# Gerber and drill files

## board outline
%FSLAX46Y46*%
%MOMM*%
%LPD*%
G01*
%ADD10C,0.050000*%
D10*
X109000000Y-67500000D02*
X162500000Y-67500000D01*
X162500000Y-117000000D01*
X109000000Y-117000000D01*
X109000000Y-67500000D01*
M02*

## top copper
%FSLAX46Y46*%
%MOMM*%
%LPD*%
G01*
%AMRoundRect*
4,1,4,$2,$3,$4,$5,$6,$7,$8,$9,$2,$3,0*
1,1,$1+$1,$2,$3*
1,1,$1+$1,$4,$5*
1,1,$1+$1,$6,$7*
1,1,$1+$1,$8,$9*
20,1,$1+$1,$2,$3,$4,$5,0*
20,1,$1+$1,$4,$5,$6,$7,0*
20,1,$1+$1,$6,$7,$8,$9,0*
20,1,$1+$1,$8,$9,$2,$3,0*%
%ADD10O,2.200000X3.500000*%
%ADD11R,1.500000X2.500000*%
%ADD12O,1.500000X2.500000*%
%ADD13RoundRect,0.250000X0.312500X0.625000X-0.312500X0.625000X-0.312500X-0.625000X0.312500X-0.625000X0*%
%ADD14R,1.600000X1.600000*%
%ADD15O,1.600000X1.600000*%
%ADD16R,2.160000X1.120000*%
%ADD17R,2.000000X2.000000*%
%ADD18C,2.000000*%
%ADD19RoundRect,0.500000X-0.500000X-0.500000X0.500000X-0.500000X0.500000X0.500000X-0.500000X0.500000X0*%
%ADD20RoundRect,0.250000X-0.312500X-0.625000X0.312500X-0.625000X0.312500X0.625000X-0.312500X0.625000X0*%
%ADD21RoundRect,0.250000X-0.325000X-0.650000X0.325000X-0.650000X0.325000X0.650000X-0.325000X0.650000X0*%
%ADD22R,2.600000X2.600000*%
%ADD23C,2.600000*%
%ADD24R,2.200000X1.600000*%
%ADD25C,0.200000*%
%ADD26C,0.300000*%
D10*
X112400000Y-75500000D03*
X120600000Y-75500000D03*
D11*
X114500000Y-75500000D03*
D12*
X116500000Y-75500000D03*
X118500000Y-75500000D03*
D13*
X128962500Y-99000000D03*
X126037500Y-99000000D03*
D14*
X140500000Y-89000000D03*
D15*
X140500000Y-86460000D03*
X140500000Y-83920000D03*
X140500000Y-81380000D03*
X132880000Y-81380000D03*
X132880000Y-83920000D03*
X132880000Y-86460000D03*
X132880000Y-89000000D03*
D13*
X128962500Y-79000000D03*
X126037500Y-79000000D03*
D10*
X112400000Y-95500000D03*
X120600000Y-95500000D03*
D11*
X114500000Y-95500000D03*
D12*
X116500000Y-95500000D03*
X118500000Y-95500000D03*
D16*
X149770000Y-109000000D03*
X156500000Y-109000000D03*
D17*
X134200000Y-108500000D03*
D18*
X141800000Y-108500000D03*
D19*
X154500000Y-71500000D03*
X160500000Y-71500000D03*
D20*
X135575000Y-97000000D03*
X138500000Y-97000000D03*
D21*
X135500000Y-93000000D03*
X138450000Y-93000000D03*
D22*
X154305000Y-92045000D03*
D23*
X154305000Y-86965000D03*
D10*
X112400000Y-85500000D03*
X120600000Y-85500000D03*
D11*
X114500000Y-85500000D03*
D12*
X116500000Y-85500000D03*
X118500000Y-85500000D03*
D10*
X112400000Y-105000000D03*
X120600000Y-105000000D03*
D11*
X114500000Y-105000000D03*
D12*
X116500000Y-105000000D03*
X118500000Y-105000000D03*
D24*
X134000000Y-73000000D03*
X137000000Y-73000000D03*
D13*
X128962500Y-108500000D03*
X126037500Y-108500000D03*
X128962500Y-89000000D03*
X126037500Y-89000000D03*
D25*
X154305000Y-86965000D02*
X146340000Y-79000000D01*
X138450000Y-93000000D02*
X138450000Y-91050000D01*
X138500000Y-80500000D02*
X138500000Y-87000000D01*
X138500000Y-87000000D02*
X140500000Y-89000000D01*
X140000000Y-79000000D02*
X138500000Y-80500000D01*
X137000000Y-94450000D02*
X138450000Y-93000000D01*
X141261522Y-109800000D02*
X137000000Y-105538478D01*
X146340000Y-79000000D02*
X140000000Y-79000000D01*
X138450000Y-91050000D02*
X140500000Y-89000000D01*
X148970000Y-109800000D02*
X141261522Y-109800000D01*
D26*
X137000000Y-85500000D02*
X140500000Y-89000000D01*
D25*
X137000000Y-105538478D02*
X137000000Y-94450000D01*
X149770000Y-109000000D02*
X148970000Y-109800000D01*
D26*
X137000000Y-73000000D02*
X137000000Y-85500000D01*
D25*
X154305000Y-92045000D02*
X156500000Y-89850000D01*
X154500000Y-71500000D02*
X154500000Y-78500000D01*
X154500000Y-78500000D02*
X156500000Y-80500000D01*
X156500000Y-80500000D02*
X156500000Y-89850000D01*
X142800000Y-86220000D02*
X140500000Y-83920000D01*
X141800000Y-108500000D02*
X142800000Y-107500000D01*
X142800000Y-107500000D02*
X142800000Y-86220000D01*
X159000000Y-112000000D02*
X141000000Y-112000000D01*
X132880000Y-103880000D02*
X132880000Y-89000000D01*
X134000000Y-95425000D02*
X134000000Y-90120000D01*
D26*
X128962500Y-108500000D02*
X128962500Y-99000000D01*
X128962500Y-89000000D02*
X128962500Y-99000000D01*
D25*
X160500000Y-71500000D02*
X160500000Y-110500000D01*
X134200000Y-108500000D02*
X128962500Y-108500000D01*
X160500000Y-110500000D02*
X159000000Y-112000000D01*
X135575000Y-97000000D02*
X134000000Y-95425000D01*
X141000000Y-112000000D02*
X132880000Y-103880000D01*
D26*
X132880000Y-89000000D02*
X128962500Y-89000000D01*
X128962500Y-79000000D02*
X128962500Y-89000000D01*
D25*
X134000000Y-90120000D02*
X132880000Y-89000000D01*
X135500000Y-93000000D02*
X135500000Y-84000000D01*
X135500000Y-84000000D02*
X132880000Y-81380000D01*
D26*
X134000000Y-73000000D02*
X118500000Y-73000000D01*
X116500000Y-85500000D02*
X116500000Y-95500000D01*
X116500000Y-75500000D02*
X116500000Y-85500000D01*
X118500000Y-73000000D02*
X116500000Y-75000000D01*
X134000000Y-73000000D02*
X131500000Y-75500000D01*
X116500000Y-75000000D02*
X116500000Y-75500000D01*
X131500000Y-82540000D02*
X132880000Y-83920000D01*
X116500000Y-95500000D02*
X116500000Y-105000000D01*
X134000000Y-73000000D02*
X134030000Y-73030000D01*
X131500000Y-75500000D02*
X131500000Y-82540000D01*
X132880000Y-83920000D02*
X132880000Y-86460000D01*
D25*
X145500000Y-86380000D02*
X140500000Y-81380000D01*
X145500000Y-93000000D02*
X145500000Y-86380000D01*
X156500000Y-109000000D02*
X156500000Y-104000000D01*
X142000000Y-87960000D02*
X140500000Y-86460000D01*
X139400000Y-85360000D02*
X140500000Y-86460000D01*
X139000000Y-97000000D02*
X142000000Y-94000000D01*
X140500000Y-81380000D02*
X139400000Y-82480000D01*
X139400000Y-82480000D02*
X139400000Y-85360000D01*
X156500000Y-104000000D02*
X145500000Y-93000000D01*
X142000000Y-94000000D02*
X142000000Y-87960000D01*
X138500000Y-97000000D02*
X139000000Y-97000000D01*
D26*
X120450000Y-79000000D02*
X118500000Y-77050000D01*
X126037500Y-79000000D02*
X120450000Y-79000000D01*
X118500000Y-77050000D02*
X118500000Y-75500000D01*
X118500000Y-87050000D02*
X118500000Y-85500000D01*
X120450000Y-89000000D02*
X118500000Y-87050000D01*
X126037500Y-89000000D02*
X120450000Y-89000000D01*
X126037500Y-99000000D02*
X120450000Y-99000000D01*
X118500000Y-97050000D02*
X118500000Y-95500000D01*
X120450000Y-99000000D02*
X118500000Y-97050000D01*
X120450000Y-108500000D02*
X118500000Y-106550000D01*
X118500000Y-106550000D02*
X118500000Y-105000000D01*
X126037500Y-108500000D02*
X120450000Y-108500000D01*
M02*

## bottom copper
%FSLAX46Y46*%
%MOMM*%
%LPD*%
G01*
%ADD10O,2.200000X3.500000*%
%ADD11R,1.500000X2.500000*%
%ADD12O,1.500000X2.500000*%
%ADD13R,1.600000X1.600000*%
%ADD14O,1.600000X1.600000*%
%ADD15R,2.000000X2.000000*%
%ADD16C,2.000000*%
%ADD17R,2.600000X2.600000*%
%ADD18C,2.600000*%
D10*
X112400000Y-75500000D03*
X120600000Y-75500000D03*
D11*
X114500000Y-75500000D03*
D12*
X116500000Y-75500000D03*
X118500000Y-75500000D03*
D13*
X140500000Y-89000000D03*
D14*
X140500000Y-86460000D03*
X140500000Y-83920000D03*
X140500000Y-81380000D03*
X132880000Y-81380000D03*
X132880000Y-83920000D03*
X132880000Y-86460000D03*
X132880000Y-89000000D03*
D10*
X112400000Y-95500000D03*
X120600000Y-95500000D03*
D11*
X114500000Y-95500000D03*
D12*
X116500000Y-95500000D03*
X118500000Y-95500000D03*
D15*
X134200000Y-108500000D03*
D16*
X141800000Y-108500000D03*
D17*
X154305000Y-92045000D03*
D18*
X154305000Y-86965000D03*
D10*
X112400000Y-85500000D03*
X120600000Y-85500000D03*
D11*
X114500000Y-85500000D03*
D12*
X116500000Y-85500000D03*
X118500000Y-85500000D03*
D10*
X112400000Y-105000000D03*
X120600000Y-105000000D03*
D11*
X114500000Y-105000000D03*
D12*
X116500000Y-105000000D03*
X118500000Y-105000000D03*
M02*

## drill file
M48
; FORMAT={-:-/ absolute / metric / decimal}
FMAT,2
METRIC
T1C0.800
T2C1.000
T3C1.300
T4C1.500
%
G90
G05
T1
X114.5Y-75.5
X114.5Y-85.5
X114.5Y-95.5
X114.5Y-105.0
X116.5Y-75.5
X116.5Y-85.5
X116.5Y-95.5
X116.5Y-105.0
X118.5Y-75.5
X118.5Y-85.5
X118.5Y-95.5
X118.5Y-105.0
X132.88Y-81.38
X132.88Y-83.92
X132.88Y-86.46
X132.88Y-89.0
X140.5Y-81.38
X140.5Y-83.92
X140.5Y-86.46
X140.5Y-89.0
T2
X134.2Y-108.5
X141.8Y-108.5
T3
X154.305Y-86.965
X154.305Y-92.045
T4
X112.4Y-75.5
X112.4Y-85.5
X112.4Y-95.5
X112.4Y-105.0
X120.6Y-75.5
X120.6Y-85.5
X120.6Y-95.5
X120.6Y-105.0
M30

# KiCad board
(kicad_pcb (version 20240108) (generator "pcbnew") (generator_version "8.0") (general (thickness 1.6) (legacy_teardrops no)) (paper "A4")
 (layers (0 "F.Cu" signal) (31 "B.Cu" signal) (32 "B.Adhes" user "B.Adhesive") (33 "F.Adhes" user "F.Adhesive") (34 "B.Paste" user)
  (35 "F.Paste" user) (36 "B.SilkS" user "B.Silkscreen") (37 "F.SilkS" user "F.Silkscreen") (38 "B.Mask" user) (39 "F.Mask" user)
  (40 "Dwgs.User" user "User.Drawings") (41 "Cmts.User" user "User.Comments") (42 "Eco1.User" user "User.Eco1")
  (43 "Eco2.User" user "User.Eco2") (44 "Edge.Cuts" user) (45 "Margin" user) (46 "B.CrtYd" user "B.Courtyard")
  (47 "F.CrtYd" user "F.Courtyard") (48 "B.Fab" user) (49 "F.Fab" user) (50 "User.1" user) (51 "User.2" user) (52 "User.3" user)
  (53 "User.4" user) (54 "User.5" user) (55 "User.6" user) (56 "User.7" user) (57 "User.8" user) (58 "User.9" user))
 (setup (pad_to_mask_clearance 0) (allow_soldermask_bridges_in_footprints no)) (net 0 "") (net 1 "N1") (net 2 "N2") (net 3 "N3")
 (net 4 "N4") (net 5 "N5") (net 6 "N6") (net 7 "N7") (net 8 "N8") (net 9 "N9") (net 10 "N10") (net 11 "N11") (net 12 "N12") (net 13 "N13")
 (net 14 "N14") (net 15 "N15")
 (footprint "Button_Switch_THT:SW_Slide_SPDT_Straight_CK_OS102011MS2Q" (layer "F.Cu") (at 114.5 75.5)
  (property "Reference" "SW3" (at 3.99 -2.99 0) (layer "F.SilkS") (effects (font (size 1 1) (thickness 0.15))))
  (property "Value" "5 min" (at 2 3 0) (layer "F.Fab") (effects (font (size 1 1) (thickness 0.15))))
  (pad "" thru_hole oval (at -2.1 0) (size 2.2 3.5) (drill 1.5) (layers "*.Cu" "*.Mask") (remove_unused_layers no))
  (pad "" thru_hole oval (at 6.1 0) (size 2.2 3.5) (drill 1.5) (layers "*.Cu" "*.Mask") (remove_unused_layers no))
  (pad "1" thru_hole rect (at 0 0) (size 1.5 2.5) (drill 0.8) (layers "*.Cu" "*.Mask") (remove_unused_layers no) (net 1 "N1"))
  (pad "2" thru_hole oval (at 2 0) (size 1.5 2.5) (drill 0.8) (layers "*.Cu" "*.Mask") (remove_unused_layers no) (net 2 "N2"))
  (pad "3" thru_hole oval (at 4 0) (size 1.5 2.5) (drill 0.8) (layers "*.Cu" "*.Mask") (remove_unused_layers no) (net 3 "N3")))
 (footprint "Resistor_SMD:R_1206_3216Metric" (layer "F.Cu") (at 127.5 99 180)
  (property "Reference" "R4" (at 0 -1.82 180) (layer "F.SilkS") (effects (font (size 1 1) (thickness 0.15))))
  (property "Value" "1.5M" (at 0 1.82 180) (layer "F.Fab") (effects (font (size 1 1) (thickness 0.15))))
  (pad "1" smd roundrect (at -1.4625 0 180) (size 1.125 1.75) (layers "F.Cu" "F.Paste" "F.Mask") (roundrect_rratio 0.222222) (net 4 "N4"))
  (pad "2" smd roundrect (at 1.4625 0 180) (size 1.125 1.75) (layers "F.Cu" "F.Paste" "F.Mask") (roundrect_rratio 0.222222) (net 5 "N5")))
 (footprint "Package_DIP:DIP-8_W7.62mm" (layer "F.Cu") (at 140.5 89 180)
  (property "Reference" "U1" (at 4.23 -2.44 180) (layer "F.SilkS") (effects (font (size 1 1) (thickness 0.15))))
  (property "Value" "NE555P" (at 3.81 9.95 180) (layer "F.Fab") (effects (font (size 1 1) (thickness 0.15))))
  (pad "1" thru_hole rect (at 0 0 180) (size 1.6 1.6) (drill 0.8) (layers "*.Cu" "*.Mask") (remove_unused_layers no) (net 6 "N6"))
  (pad "2" thru_hole oval (at 0 2.54 180) (size 1.6 1.6) (drill 0.8) (layers "*.Cu" "*.Mask") (remove_unused_layers no) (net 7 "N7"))
  (pad "3" thru_hole oval (at 0 5.08 180) (size 1.6 1.6) (drill 0.8) (layers "*.Cu" "*.Mask") (remove_unused_layers no) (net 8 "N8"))
  (pad "4" thru_hole oval (at 0 7.62 180) (size 1.6 1.6) (drill 0.8) (layers "*.Cu" "*.Mask") (remove_unused_layers no) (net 7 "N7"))
  (pad "5" thru_hole oval (at 7.62 7.62 180) (size 1.6 1.6) (drill 0.8) (layers "*.Cu" "*.Mask") (remove_unused_layers no) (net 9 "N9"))
  (pad "6" thru_hole oval (at 7.62 5.08 180) (size 1.6 1.6) (drill 0.8) (layers "*.Cu" "*.Mask") (remove_unused_layers no) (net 2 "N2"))
  (pad "7" thru_hole oval (at 7.62 2.54 180) (size 1.6 1.6) (drill 0.8) (layers "*.Cu" "*.Mask") (remove_unused_layers no) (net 2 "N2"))
  (pad "8" thru_hole oval (at 7.62 0 180) (size 1.6 1.6) (drill 0.8) (layers "*.Cu" "*.Mask") (remove_unused_layers no) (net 4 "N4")))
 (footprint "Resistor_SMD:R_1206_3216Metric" (layer "F.Cu") (at 127.5 79 180)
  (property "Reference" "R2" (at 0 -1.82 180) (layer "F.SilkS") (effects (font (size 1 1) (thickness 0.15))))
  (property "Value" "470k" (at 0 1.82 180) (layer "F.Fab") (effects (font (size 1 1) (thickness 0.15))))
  (pad "1" smd roundrect (at -1.4625 0 180) (size 1.125 1.75) (layers "F.Cu" "F.Paste" "F.Mask") (roundrect_rratio 0.222222) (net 4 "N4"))
  (pad "2" smd roundrect (at 1.4625 0 180) (size 1.125 1.75) (layers "F.Cu" "F.Paste" "F.Mask") (roundrect_rratio 0.222222) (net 3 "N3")))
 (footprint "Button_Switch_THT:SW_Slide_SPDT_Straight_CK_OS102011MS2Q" (layer "F.Cu") (at 114.5 95.5)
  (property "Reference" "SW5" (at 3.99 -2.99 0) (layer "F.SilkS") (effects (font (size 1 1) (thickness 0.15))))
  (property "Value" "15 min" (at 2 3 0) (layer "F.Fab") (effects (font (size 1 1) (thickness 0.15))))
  (pad "" thru_hole oval (at -2.1 0) (size 2.2 3.5) (drill 1.5) (layers "*.Cu" "*.Mask") (remove_unused_layers no))
  (pad "" thru_hole oval (at 6.1 0) (size 2.2 3.5) (drill 1.5) (layers "*.Cu" "*.Mask") (remove_unused_layers no))
  (pad "1" thru_hole rect (at 0 0) (size 1.5 2.5) (drill 0.8) (layers "*.Cu" "*.Mask") (remove_unused_layers no) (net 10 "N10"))
  (pad "2" thru_hole oval (at 2 0) (size 1.5 2.5) (drill 0.8) (layers "*.Cu" "*.Mask") (remove_unused_layers no) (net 2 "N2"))
  (pad "3" thru_hole oval (at 4 0) (size 1.5 2.5) (drill 0.8) (layers "*.Cu" "*.Mask") (remove_unused_layers no) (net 5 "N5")))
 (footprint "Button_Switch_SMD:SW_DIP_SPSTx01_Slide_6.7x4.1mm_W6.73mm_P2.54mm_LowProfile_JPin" (layer "F.Cu") (at 153.135 109)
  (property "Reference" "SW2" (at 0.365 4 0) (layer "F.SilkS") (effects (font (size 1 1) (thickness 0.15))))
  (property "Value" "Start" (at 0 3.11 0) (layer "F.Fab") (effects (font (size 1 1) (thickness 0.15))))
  (pad "1" smd rect (at -3.365 0) (size 2.16 1.12) (layers "F.Cu" "F.Paste" "F.Mask") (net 6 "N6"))
  (pad "2" smd rect (at 3.365 0) (size 2.16 1.12) (layers "F.Cu" "F.Paste" "F.Mask") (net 7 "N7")))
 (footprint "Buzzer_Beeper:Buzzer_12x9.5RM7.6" (layer "F.Cu") (at 134.2 108.5)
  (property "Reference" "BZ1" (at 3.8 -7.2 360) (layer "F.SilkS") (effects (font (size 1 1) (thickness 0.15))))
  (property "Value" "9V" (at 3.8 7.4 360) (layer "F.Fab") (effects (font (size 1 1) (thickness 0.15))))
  (pad "1" thru_hole rect (at 0 0) (size 2 2) (drill 1) (layers "*.Cu" "*.Mask") (remove_unused_layers no) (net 4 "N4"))
  (pad "2" thru_hole circle (at 7.6 0) (size 2 2) (drill 1) (layers "*.Cu" "*.Mask") (remove_unused_layers no) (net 8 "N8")))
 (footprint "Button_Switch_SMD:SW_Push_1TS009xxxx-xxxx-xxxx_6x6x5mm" (layer "F.Cu") (at 157.5 71.5)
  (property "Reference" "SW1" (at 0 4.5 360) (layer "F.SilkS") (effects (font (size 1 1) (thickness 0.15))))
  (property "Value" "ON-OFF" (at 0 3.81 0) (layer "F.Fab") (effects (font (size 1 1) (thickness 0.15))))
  (pad "1" smd roundrect (at -3 0) (size 2 2) (layers "F.Cu" "F.Paste" "F.Mask") (roundrect_rratio 0.25) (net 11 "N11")
   (thermal_bridge_angle 45))
  (pad "2" smd roundrect (at 3 0) (size 2 2) (layers "F.Cu" "F.Paste" "F.Mask") (roundrect_rratio 0.25) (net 4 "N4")
   (thermal_bridge_angle 45)))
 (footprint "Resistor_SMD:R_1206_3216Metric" (layer "F.Cu") (at 137.0375 97)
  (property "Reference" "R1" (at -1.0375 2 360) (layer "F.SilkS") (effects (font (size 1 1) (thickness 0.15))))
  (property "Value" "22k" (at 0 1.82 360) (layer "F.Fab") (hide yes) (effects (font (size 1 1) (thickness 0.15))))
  (pad "1" smd roundrect (at -1.4625 0) (size 1.125 1.75) (layers "F.Cu" "F.Paste" "F.Mask") (roundrect_rratio 0.222222) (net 4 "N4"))
  (pad "2" smd roundrect (at 1.4625 0) (size 1.125 1.75) (layers "F.Cu" "F.Paste" "F.Mask") (roundrect_rratio 0.222222) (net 7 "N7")))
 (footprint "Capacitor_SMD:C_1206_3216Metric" (layer "F.Cu") (at 136.975 93)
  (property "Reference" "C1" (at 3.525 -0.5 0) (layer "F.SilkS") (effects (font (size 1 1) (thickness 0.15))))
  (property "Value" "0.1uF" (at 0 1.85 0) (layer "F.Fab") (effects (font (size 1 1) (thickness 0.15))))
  (pad "1" smd roundrect (at -1.475 0) (size 1.15 1.8) (layers "F.Cu" "F.Paste" "F.Mask") (roundrect_rratio 0.217391) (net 9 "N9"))
  (pad "2" smd roundrect (at 1.475 0) (size 1.15 1.8) (layers "F.Cu" "F.Paste" "F.Mask") (roundrect_rratio 0.217391) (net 6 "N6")))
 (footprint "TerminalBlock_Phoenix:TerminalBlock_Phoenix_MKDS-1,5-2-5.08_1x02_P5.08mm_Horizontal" (layer "F.Cu") (at 154.305 92.045 90)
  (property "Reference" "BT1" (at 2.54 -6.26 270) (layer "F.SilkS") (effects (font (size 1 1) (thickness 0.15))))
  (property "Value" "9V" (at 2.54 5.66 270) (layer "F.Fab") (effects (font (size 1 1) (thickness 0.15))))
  (pad "1" thru_hole rect (at 0 0 90) (size 2.6 2.6) (drill 1.3) (layers "*.Cu" "*.Mask") (remove_unused_layers no) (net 11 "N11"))
  (pad "2" thru_hole circle (at 5.08 0 90) (size 2.6 2.6) (drill 1.3) (layers "*.Cu" "*.Mask") (remove_unused_layers no) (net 6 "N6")))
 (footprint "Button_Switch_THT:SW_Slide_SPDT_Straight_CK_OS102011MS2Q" (layer "F.Cu") (at 114.5 85.5)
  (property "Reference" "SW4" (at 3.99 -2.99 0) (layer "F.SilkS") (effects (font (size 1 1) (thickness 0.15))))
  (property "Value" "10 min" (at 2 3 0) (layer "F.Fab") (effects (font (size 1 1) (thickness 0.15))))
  (pad "" thru_hole oval (at -2.1 0) (size 2.2 3.5) (drill 1.5) (layers "*.Cu" "*.Mask") (remove_unused_layers no))
  (pad "" thru_hole oval (at 6.1 0) (size 2.2 3.5) (drill 1.5) (layers "*.Cu" "*.Mask") (remove_unused_layers no))
  (pad "1" thru_hole rect (at 0 0) (size 1.5 2.5) (drill 0.8) (layers "*.Cu" "*.Mask") (remove_unused_layers no) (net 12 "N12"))
  (pad "2" thru_hole oval (at 2 0) (size 1.5 2.5) (drill 0.8) (layers "*.Cu" "*.Mask") (remove_unused_layers no) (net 2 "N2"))
  (pad "3" thru_hole oval (at 4 0) (size 1.5 2.5) (drill 0.8) (layers "*.Cu" "*.Mask") (remove_unused_layers no) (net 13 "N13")))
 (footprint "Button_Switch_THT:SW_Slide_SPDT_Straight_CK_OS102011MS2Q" (layer "F.Cu") (at 114.5 105)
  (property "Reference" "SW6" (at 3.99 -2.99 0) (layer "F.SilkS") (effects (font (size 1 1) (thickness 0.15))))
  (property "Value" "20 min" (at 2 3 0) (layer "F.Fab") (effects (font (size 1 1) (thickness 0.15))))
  (pad "" thru_hole oval (at -2.1 0) (size 2.2 3.5) (drill 1.5) (layers "*.Cu" "*.Mask") (remove_unused_layers no))
  (pad "" thru_hole oval (at 6.1 0) (size 2.2 3.5) (drill 1.5) (layers "*.Cu" "*.Mask") (remove_unused_layers no))
  (pad "1" thru_hole rect (at 0 0) (size 1.5 2.5) (drill 0.8) (layers "*.Cu" "*.Mask") (remove_unused_layers no) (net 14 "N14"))
  (pad "2" thru_hole oval (at 2 0) (size 1.5 2.5) (drill 0.8) (layers "*.Cu" "*.Mask") (remove_unused_layers no) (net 2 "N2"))
  (pad "3" thru_hole oval (at 4 0) (size 1.5 2.5) (drill 0.8) (layers "*.Cu" "*.Mask") (remove_unused_layers no) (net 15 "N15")))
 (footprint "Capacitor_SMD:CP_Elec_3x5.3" (layer "F.Cu") (at 135.5 73)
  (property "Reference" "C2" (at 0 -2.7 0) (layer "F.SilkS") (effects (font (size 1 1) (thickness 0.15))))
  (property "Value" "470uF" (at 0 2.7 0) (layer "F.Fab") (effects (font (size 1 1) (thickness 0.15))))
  (pad "1" smd rect (at -1.5 0) (size 2.2 1.6) (layers "F.Cu" "F.Paste" "F.Mask") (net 2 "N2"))
  (pad "2" smd rect (at 1.5 0) (size 2.2 1.6) (layers "F.Cu" "F.Paste" "F.Mask") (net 6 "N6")))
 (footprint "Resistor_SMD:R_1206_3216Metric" (layer "F.Cu") (at 127.5 108.5 180)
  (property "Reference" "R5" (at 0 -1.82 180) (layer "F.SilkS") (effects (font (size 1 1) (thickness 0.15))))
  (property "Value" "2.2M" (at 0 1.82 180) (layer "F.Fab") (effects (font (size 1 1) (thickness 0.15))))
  (pad "1" smd roundrect (at -1.4625 0 180) (size 1.125 1.75) (layers "F.Cu" "F.Paste" "F.Mask") (roundrect_rratio 0.222222) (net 4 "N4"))
  (pad "2" smd roundrect (at 1.4625 0 180) (size 1.125 1.75) (layers "F.Cu" "F.Paste" "F.Mask") (roundrect_rratio 0.222222) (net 15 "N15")))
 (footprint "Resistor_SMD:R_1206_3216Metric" (layer "F.Cu") (at 127.5 89 180)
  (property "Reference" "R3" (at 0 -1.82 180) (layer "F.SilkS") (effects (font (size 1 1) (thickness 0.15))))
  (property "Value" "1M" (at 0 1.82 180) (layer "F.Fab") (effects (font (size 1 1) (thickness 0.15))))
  (pad "1" smd roundrect (at -1.4625 0 180) (size 1.125 1.75) (layers "F.Cu" "F.Paste" "F.Mask") (roundrect_rratio 0.222222) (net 4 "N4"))
  (pad "2" smd roundrect (at 1.4625 0 180) (size 1.125 1.75) (layers "F.Cu" "F.Paste" "F.Mask") (roundrect_rratio 0.222222) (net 13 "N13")))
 (gr_rect (start 109 67.5) (end 162.5 117) (stroke (width 0.05) (type default)) (fill none) (layer "Edge.Cuts"))
 (segment (start 154.305 86.965) (end 146.34 79) (width 0.2) (layer "F.Cu") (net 6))
 (segment (start 138.45 93) (end 138.45 91.05) (width 0.2) (layer "F.Cu") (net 6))
 (segment (start 138.5 80.5) (end 138.5 87) (width 0.2) (layer "F.Cu") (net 6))
 (segment (start 138.5 87) (end 140.5 89) (width 0.2) (layer "F.Cu") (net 6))
 (segment (start 140 79) (end 138.5 80.5) (width 0.2) (layer "F.Cu") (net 6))
 (segment (start 137 94.45) (end 138.45 93) (width 0.2) (layer "F.Cu") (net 6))
 (segment (start 141.261522 109.8) (end 137 105.538478) (width 0.2) (layer "F.Cu") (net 6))
 (segment (start 146.34 79) (end 140 79) (width 0.2) (layer "F.Cu") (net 6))
 (segment (start 138.45 91.05) (end 140.5 89) (width 0.2) (layer "F.Cu") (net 6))
 (segment (start 148.97 109.8) (end 141.261522 109.8) (width 0.2) (layer "F.Cu") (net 6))
 (segment (start 137 85.5) (end 140.5 89) (width 0.3) (layer "F.Cu") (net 6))
 (segment (start 137 105.538478) (end 137 94.45) (width 0.2) (layer "F.Cu") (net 6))
 (segment (start 149.77 109) (end 148.97 109.8) (width 0.2) (layer "F.Cu") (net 6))
 (segment (start 137 73) (end 137 85.5) (width 0.3) (layer "F.Cu") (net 6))
 (segment (start 154.305 92.045) (end 156.5 89.85) (width 0.2) (layer "F.Cu") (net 11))
 (segment (start 154.5 71.5) (end 154.5 78.5) (width 0.2) (layer "F.Cu") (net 11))
 (segment (start 154.5 78.5) (end 156.5 80.5) (width 0.2) (layer "F.Cu") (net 11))
 (segment (start 156.5 80.5) (end 156.5 89.85) (width 0.2) (layer "F.Cu") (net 11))
 (segment (start 142.8 86.22) (end 140.5 83.92) (width 0.2) (layer "F.Cu") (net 8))
 (segment (start 141.8 108.5) (end 142.8 107.5) (width 0.2) (layer "F.Cu") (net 8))
 (segment (start 142.8 107.5) (end 142.8 86.22) (width 0.2) (layer "F.Cu") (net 8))
 (segment (start 159 112) (end 141 112) (width 0.2) (layer "F.Cu") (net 4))
 (segment (start 132.88 103.88) (end 132.88 89) (width 0.2) (layer "F.Cu") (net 4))
 (segment (start 134 95.425) (end 134 90.12) (width 0.2) (layer "F.Cu") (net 4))
 (segment (start 128.9625 108.5) (end 128.9625 99) (width 0.3) (layer "F.Cu") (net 4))
 (segment (start 128.9625 89) (end 128.9625 99) (width 0.3) (layer "F.Cu") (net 4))
 (segment (start 160.5 71.5) (end 160.5 110.5) (width 0.2) (layer "F.Cu") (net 4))
 (segment (start 134.2 108.5) (end 128.9625 108.5) (width 0.2) (layer "F.Cu") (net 4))
 (segment (start 160.5 110.5) (end 159 112) (width 0.2) (layer "F.Cu") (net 4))
 (segment (start 135.575 97) (end 134 95.425) (width 0.2) (layer "F.Cu") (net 4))
 (segment (start 141 112) (end 132.88 103.88) (width 0.2) (layer "F.Cu") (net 4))
 (segment (start 132.88 89) (end 128.9625 89) (width 0.3) (layer "F.Cu") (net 4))
 (segment (start 128.9625 79) (end 128.9625 89) (width 0.3) (layer "F.Cu") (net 4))
 (segment (start 134 90.12) (end 132.88 89) (width 0.2) (layer "F.Cu") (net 4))
 (segment (start 135.5 93) (end 135.5 84) (width 0.2) (layer "F.Cu") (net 9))
 (segment (start 135.5 84) (end 132.88 81.38) (width 0.2) (layer "F.Cu") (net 9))
 (segment (start 134 73) (end 118.5 73) (width 0.3) (layer "F.Cu") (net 2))
 (segment (start 116.5 85.5) (end 116.5 95.5) (width 0.3) (layer "F.Cu") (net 2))
 (segment (start 116.5 75.5) (end 116.5 85.5) (width 0.3) (layer "F.Cu") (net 2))
 (segment (start 118.5 73) (end 116.5 75) (width 0.3) (layer "F.Cu") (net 2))
 (segment (start 134 73) (end 131.5 75.5) (width 0.3) (layer "F.Cu") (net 2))
 (segment (start 116.5 75) (end 116.5 75.5) (width 0.3) (layer "F.Cu") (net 2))
 (segment (start 131.5 82.54) (end 132.88 83.92) (width 0.3) (layer "F.Cu") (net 2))
 (segment (start 116.5 95.5) (end 116.5 105) (width 0.3) (layer "F.Cu") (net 2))
 (segment (start 134 73) (end 134.03 73.03) (width 0.3) (layer "F.Cu") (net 2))
 (segment (start 131.5 75.5) (end 131.5 82.54) (width 0.3) (layer "F.Cu") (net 2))
 (segment (start 132.88 83.92) (end 132.88 86.46) (width 0.3) (layer "F.Cu") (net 2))
 (segment (start 145.5 86.38) (end 140.5 81.38) (width 0.2) (layer "F.Cu") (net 7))
 (segment (start 145.5 93) (end 145.5 86.38) (width 0.2) (layer "F.Cu") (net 7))
 (segment (start 156.5 109) (end 156.5 104) (width 0.2) (layer "F.Cu") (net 7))
 (segment (start 142 87.96) (end 140.5 86.46) (width 0.2) (layer "F.Cu") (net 7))
 (segment (start 139.4 85.36) (end 140.5 86.46) (width 0.2) (layer "F.Cu") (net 7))
 (segment (start 139 97) (end 142 94) (width 0.2) (layer "F.Cu") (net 7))
 (segment (start 140.5 81.38) (end 139.4 82.48) (width 0.2) (layer "F.Cu") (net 7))
 (segment (start 139.4 82.48) (end 139.4 85.36) (width 0.2) (layer "F.Cu") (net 7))
 (segment (start 156.5 104) (end 145.5 93) (width 0.2) (layer "F.Cu") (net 7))
 (segment (start 142 94) (end 142 87.96) (width 0.2) (layer "F.Cu") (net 7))
 (segment (start 138.5 97) (end 139 97) (width 0.2) (layer "F.Cu") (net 7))
 (segment (start 120.45 79) (end 118.5 77.05) (width 0.3) (layer "F.Cu") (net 3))
 (segment (start 126.0375 79) (end 120.45 79) (width 0.3) (layer "F.Cu") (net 3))
 (segment (start 118.5 77.05) (end 118.5 75.5) (width 0.3) (layer "F.Cu") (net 3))
 (segment (start 118.5 87.05) (end 118.5 85.5) (width 0.3) (layer "F.Cu") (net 13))
 (segment (start 120.45 89) (end 118.5 87.05) (width 0.3) (layer "F.Cu") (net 13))
 (segment (start 126.0375 89) (end 120.45 89) (width 0.3) (layer "F.Cu") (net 13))
 (segment (start 126.0375 99) (end 120.45 99) (width 0.3) (layer "F.Cu") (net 5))
 (segment (start 118.5 97.05) (end 118.5 95.5) (width 0.3) (layer "F.Cu") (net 5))
 (segment (start 120.45 99) (end 118.5 97.05) (width 0.3) (layer "F.Cu") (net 5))
 (segment (start 120.45 108.5) (end 118.5 106.55) (width 0.3) (layer "F.Cu") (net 15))
 (segment (start 118.5 106.55) (end 118.5 105) (width 0.3) (layer "F.Cu") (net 15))
 (segment (start 126.0375 108.5) (end 120.45 108.5) (width 0.3) (layer "F.Cu") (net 15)))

